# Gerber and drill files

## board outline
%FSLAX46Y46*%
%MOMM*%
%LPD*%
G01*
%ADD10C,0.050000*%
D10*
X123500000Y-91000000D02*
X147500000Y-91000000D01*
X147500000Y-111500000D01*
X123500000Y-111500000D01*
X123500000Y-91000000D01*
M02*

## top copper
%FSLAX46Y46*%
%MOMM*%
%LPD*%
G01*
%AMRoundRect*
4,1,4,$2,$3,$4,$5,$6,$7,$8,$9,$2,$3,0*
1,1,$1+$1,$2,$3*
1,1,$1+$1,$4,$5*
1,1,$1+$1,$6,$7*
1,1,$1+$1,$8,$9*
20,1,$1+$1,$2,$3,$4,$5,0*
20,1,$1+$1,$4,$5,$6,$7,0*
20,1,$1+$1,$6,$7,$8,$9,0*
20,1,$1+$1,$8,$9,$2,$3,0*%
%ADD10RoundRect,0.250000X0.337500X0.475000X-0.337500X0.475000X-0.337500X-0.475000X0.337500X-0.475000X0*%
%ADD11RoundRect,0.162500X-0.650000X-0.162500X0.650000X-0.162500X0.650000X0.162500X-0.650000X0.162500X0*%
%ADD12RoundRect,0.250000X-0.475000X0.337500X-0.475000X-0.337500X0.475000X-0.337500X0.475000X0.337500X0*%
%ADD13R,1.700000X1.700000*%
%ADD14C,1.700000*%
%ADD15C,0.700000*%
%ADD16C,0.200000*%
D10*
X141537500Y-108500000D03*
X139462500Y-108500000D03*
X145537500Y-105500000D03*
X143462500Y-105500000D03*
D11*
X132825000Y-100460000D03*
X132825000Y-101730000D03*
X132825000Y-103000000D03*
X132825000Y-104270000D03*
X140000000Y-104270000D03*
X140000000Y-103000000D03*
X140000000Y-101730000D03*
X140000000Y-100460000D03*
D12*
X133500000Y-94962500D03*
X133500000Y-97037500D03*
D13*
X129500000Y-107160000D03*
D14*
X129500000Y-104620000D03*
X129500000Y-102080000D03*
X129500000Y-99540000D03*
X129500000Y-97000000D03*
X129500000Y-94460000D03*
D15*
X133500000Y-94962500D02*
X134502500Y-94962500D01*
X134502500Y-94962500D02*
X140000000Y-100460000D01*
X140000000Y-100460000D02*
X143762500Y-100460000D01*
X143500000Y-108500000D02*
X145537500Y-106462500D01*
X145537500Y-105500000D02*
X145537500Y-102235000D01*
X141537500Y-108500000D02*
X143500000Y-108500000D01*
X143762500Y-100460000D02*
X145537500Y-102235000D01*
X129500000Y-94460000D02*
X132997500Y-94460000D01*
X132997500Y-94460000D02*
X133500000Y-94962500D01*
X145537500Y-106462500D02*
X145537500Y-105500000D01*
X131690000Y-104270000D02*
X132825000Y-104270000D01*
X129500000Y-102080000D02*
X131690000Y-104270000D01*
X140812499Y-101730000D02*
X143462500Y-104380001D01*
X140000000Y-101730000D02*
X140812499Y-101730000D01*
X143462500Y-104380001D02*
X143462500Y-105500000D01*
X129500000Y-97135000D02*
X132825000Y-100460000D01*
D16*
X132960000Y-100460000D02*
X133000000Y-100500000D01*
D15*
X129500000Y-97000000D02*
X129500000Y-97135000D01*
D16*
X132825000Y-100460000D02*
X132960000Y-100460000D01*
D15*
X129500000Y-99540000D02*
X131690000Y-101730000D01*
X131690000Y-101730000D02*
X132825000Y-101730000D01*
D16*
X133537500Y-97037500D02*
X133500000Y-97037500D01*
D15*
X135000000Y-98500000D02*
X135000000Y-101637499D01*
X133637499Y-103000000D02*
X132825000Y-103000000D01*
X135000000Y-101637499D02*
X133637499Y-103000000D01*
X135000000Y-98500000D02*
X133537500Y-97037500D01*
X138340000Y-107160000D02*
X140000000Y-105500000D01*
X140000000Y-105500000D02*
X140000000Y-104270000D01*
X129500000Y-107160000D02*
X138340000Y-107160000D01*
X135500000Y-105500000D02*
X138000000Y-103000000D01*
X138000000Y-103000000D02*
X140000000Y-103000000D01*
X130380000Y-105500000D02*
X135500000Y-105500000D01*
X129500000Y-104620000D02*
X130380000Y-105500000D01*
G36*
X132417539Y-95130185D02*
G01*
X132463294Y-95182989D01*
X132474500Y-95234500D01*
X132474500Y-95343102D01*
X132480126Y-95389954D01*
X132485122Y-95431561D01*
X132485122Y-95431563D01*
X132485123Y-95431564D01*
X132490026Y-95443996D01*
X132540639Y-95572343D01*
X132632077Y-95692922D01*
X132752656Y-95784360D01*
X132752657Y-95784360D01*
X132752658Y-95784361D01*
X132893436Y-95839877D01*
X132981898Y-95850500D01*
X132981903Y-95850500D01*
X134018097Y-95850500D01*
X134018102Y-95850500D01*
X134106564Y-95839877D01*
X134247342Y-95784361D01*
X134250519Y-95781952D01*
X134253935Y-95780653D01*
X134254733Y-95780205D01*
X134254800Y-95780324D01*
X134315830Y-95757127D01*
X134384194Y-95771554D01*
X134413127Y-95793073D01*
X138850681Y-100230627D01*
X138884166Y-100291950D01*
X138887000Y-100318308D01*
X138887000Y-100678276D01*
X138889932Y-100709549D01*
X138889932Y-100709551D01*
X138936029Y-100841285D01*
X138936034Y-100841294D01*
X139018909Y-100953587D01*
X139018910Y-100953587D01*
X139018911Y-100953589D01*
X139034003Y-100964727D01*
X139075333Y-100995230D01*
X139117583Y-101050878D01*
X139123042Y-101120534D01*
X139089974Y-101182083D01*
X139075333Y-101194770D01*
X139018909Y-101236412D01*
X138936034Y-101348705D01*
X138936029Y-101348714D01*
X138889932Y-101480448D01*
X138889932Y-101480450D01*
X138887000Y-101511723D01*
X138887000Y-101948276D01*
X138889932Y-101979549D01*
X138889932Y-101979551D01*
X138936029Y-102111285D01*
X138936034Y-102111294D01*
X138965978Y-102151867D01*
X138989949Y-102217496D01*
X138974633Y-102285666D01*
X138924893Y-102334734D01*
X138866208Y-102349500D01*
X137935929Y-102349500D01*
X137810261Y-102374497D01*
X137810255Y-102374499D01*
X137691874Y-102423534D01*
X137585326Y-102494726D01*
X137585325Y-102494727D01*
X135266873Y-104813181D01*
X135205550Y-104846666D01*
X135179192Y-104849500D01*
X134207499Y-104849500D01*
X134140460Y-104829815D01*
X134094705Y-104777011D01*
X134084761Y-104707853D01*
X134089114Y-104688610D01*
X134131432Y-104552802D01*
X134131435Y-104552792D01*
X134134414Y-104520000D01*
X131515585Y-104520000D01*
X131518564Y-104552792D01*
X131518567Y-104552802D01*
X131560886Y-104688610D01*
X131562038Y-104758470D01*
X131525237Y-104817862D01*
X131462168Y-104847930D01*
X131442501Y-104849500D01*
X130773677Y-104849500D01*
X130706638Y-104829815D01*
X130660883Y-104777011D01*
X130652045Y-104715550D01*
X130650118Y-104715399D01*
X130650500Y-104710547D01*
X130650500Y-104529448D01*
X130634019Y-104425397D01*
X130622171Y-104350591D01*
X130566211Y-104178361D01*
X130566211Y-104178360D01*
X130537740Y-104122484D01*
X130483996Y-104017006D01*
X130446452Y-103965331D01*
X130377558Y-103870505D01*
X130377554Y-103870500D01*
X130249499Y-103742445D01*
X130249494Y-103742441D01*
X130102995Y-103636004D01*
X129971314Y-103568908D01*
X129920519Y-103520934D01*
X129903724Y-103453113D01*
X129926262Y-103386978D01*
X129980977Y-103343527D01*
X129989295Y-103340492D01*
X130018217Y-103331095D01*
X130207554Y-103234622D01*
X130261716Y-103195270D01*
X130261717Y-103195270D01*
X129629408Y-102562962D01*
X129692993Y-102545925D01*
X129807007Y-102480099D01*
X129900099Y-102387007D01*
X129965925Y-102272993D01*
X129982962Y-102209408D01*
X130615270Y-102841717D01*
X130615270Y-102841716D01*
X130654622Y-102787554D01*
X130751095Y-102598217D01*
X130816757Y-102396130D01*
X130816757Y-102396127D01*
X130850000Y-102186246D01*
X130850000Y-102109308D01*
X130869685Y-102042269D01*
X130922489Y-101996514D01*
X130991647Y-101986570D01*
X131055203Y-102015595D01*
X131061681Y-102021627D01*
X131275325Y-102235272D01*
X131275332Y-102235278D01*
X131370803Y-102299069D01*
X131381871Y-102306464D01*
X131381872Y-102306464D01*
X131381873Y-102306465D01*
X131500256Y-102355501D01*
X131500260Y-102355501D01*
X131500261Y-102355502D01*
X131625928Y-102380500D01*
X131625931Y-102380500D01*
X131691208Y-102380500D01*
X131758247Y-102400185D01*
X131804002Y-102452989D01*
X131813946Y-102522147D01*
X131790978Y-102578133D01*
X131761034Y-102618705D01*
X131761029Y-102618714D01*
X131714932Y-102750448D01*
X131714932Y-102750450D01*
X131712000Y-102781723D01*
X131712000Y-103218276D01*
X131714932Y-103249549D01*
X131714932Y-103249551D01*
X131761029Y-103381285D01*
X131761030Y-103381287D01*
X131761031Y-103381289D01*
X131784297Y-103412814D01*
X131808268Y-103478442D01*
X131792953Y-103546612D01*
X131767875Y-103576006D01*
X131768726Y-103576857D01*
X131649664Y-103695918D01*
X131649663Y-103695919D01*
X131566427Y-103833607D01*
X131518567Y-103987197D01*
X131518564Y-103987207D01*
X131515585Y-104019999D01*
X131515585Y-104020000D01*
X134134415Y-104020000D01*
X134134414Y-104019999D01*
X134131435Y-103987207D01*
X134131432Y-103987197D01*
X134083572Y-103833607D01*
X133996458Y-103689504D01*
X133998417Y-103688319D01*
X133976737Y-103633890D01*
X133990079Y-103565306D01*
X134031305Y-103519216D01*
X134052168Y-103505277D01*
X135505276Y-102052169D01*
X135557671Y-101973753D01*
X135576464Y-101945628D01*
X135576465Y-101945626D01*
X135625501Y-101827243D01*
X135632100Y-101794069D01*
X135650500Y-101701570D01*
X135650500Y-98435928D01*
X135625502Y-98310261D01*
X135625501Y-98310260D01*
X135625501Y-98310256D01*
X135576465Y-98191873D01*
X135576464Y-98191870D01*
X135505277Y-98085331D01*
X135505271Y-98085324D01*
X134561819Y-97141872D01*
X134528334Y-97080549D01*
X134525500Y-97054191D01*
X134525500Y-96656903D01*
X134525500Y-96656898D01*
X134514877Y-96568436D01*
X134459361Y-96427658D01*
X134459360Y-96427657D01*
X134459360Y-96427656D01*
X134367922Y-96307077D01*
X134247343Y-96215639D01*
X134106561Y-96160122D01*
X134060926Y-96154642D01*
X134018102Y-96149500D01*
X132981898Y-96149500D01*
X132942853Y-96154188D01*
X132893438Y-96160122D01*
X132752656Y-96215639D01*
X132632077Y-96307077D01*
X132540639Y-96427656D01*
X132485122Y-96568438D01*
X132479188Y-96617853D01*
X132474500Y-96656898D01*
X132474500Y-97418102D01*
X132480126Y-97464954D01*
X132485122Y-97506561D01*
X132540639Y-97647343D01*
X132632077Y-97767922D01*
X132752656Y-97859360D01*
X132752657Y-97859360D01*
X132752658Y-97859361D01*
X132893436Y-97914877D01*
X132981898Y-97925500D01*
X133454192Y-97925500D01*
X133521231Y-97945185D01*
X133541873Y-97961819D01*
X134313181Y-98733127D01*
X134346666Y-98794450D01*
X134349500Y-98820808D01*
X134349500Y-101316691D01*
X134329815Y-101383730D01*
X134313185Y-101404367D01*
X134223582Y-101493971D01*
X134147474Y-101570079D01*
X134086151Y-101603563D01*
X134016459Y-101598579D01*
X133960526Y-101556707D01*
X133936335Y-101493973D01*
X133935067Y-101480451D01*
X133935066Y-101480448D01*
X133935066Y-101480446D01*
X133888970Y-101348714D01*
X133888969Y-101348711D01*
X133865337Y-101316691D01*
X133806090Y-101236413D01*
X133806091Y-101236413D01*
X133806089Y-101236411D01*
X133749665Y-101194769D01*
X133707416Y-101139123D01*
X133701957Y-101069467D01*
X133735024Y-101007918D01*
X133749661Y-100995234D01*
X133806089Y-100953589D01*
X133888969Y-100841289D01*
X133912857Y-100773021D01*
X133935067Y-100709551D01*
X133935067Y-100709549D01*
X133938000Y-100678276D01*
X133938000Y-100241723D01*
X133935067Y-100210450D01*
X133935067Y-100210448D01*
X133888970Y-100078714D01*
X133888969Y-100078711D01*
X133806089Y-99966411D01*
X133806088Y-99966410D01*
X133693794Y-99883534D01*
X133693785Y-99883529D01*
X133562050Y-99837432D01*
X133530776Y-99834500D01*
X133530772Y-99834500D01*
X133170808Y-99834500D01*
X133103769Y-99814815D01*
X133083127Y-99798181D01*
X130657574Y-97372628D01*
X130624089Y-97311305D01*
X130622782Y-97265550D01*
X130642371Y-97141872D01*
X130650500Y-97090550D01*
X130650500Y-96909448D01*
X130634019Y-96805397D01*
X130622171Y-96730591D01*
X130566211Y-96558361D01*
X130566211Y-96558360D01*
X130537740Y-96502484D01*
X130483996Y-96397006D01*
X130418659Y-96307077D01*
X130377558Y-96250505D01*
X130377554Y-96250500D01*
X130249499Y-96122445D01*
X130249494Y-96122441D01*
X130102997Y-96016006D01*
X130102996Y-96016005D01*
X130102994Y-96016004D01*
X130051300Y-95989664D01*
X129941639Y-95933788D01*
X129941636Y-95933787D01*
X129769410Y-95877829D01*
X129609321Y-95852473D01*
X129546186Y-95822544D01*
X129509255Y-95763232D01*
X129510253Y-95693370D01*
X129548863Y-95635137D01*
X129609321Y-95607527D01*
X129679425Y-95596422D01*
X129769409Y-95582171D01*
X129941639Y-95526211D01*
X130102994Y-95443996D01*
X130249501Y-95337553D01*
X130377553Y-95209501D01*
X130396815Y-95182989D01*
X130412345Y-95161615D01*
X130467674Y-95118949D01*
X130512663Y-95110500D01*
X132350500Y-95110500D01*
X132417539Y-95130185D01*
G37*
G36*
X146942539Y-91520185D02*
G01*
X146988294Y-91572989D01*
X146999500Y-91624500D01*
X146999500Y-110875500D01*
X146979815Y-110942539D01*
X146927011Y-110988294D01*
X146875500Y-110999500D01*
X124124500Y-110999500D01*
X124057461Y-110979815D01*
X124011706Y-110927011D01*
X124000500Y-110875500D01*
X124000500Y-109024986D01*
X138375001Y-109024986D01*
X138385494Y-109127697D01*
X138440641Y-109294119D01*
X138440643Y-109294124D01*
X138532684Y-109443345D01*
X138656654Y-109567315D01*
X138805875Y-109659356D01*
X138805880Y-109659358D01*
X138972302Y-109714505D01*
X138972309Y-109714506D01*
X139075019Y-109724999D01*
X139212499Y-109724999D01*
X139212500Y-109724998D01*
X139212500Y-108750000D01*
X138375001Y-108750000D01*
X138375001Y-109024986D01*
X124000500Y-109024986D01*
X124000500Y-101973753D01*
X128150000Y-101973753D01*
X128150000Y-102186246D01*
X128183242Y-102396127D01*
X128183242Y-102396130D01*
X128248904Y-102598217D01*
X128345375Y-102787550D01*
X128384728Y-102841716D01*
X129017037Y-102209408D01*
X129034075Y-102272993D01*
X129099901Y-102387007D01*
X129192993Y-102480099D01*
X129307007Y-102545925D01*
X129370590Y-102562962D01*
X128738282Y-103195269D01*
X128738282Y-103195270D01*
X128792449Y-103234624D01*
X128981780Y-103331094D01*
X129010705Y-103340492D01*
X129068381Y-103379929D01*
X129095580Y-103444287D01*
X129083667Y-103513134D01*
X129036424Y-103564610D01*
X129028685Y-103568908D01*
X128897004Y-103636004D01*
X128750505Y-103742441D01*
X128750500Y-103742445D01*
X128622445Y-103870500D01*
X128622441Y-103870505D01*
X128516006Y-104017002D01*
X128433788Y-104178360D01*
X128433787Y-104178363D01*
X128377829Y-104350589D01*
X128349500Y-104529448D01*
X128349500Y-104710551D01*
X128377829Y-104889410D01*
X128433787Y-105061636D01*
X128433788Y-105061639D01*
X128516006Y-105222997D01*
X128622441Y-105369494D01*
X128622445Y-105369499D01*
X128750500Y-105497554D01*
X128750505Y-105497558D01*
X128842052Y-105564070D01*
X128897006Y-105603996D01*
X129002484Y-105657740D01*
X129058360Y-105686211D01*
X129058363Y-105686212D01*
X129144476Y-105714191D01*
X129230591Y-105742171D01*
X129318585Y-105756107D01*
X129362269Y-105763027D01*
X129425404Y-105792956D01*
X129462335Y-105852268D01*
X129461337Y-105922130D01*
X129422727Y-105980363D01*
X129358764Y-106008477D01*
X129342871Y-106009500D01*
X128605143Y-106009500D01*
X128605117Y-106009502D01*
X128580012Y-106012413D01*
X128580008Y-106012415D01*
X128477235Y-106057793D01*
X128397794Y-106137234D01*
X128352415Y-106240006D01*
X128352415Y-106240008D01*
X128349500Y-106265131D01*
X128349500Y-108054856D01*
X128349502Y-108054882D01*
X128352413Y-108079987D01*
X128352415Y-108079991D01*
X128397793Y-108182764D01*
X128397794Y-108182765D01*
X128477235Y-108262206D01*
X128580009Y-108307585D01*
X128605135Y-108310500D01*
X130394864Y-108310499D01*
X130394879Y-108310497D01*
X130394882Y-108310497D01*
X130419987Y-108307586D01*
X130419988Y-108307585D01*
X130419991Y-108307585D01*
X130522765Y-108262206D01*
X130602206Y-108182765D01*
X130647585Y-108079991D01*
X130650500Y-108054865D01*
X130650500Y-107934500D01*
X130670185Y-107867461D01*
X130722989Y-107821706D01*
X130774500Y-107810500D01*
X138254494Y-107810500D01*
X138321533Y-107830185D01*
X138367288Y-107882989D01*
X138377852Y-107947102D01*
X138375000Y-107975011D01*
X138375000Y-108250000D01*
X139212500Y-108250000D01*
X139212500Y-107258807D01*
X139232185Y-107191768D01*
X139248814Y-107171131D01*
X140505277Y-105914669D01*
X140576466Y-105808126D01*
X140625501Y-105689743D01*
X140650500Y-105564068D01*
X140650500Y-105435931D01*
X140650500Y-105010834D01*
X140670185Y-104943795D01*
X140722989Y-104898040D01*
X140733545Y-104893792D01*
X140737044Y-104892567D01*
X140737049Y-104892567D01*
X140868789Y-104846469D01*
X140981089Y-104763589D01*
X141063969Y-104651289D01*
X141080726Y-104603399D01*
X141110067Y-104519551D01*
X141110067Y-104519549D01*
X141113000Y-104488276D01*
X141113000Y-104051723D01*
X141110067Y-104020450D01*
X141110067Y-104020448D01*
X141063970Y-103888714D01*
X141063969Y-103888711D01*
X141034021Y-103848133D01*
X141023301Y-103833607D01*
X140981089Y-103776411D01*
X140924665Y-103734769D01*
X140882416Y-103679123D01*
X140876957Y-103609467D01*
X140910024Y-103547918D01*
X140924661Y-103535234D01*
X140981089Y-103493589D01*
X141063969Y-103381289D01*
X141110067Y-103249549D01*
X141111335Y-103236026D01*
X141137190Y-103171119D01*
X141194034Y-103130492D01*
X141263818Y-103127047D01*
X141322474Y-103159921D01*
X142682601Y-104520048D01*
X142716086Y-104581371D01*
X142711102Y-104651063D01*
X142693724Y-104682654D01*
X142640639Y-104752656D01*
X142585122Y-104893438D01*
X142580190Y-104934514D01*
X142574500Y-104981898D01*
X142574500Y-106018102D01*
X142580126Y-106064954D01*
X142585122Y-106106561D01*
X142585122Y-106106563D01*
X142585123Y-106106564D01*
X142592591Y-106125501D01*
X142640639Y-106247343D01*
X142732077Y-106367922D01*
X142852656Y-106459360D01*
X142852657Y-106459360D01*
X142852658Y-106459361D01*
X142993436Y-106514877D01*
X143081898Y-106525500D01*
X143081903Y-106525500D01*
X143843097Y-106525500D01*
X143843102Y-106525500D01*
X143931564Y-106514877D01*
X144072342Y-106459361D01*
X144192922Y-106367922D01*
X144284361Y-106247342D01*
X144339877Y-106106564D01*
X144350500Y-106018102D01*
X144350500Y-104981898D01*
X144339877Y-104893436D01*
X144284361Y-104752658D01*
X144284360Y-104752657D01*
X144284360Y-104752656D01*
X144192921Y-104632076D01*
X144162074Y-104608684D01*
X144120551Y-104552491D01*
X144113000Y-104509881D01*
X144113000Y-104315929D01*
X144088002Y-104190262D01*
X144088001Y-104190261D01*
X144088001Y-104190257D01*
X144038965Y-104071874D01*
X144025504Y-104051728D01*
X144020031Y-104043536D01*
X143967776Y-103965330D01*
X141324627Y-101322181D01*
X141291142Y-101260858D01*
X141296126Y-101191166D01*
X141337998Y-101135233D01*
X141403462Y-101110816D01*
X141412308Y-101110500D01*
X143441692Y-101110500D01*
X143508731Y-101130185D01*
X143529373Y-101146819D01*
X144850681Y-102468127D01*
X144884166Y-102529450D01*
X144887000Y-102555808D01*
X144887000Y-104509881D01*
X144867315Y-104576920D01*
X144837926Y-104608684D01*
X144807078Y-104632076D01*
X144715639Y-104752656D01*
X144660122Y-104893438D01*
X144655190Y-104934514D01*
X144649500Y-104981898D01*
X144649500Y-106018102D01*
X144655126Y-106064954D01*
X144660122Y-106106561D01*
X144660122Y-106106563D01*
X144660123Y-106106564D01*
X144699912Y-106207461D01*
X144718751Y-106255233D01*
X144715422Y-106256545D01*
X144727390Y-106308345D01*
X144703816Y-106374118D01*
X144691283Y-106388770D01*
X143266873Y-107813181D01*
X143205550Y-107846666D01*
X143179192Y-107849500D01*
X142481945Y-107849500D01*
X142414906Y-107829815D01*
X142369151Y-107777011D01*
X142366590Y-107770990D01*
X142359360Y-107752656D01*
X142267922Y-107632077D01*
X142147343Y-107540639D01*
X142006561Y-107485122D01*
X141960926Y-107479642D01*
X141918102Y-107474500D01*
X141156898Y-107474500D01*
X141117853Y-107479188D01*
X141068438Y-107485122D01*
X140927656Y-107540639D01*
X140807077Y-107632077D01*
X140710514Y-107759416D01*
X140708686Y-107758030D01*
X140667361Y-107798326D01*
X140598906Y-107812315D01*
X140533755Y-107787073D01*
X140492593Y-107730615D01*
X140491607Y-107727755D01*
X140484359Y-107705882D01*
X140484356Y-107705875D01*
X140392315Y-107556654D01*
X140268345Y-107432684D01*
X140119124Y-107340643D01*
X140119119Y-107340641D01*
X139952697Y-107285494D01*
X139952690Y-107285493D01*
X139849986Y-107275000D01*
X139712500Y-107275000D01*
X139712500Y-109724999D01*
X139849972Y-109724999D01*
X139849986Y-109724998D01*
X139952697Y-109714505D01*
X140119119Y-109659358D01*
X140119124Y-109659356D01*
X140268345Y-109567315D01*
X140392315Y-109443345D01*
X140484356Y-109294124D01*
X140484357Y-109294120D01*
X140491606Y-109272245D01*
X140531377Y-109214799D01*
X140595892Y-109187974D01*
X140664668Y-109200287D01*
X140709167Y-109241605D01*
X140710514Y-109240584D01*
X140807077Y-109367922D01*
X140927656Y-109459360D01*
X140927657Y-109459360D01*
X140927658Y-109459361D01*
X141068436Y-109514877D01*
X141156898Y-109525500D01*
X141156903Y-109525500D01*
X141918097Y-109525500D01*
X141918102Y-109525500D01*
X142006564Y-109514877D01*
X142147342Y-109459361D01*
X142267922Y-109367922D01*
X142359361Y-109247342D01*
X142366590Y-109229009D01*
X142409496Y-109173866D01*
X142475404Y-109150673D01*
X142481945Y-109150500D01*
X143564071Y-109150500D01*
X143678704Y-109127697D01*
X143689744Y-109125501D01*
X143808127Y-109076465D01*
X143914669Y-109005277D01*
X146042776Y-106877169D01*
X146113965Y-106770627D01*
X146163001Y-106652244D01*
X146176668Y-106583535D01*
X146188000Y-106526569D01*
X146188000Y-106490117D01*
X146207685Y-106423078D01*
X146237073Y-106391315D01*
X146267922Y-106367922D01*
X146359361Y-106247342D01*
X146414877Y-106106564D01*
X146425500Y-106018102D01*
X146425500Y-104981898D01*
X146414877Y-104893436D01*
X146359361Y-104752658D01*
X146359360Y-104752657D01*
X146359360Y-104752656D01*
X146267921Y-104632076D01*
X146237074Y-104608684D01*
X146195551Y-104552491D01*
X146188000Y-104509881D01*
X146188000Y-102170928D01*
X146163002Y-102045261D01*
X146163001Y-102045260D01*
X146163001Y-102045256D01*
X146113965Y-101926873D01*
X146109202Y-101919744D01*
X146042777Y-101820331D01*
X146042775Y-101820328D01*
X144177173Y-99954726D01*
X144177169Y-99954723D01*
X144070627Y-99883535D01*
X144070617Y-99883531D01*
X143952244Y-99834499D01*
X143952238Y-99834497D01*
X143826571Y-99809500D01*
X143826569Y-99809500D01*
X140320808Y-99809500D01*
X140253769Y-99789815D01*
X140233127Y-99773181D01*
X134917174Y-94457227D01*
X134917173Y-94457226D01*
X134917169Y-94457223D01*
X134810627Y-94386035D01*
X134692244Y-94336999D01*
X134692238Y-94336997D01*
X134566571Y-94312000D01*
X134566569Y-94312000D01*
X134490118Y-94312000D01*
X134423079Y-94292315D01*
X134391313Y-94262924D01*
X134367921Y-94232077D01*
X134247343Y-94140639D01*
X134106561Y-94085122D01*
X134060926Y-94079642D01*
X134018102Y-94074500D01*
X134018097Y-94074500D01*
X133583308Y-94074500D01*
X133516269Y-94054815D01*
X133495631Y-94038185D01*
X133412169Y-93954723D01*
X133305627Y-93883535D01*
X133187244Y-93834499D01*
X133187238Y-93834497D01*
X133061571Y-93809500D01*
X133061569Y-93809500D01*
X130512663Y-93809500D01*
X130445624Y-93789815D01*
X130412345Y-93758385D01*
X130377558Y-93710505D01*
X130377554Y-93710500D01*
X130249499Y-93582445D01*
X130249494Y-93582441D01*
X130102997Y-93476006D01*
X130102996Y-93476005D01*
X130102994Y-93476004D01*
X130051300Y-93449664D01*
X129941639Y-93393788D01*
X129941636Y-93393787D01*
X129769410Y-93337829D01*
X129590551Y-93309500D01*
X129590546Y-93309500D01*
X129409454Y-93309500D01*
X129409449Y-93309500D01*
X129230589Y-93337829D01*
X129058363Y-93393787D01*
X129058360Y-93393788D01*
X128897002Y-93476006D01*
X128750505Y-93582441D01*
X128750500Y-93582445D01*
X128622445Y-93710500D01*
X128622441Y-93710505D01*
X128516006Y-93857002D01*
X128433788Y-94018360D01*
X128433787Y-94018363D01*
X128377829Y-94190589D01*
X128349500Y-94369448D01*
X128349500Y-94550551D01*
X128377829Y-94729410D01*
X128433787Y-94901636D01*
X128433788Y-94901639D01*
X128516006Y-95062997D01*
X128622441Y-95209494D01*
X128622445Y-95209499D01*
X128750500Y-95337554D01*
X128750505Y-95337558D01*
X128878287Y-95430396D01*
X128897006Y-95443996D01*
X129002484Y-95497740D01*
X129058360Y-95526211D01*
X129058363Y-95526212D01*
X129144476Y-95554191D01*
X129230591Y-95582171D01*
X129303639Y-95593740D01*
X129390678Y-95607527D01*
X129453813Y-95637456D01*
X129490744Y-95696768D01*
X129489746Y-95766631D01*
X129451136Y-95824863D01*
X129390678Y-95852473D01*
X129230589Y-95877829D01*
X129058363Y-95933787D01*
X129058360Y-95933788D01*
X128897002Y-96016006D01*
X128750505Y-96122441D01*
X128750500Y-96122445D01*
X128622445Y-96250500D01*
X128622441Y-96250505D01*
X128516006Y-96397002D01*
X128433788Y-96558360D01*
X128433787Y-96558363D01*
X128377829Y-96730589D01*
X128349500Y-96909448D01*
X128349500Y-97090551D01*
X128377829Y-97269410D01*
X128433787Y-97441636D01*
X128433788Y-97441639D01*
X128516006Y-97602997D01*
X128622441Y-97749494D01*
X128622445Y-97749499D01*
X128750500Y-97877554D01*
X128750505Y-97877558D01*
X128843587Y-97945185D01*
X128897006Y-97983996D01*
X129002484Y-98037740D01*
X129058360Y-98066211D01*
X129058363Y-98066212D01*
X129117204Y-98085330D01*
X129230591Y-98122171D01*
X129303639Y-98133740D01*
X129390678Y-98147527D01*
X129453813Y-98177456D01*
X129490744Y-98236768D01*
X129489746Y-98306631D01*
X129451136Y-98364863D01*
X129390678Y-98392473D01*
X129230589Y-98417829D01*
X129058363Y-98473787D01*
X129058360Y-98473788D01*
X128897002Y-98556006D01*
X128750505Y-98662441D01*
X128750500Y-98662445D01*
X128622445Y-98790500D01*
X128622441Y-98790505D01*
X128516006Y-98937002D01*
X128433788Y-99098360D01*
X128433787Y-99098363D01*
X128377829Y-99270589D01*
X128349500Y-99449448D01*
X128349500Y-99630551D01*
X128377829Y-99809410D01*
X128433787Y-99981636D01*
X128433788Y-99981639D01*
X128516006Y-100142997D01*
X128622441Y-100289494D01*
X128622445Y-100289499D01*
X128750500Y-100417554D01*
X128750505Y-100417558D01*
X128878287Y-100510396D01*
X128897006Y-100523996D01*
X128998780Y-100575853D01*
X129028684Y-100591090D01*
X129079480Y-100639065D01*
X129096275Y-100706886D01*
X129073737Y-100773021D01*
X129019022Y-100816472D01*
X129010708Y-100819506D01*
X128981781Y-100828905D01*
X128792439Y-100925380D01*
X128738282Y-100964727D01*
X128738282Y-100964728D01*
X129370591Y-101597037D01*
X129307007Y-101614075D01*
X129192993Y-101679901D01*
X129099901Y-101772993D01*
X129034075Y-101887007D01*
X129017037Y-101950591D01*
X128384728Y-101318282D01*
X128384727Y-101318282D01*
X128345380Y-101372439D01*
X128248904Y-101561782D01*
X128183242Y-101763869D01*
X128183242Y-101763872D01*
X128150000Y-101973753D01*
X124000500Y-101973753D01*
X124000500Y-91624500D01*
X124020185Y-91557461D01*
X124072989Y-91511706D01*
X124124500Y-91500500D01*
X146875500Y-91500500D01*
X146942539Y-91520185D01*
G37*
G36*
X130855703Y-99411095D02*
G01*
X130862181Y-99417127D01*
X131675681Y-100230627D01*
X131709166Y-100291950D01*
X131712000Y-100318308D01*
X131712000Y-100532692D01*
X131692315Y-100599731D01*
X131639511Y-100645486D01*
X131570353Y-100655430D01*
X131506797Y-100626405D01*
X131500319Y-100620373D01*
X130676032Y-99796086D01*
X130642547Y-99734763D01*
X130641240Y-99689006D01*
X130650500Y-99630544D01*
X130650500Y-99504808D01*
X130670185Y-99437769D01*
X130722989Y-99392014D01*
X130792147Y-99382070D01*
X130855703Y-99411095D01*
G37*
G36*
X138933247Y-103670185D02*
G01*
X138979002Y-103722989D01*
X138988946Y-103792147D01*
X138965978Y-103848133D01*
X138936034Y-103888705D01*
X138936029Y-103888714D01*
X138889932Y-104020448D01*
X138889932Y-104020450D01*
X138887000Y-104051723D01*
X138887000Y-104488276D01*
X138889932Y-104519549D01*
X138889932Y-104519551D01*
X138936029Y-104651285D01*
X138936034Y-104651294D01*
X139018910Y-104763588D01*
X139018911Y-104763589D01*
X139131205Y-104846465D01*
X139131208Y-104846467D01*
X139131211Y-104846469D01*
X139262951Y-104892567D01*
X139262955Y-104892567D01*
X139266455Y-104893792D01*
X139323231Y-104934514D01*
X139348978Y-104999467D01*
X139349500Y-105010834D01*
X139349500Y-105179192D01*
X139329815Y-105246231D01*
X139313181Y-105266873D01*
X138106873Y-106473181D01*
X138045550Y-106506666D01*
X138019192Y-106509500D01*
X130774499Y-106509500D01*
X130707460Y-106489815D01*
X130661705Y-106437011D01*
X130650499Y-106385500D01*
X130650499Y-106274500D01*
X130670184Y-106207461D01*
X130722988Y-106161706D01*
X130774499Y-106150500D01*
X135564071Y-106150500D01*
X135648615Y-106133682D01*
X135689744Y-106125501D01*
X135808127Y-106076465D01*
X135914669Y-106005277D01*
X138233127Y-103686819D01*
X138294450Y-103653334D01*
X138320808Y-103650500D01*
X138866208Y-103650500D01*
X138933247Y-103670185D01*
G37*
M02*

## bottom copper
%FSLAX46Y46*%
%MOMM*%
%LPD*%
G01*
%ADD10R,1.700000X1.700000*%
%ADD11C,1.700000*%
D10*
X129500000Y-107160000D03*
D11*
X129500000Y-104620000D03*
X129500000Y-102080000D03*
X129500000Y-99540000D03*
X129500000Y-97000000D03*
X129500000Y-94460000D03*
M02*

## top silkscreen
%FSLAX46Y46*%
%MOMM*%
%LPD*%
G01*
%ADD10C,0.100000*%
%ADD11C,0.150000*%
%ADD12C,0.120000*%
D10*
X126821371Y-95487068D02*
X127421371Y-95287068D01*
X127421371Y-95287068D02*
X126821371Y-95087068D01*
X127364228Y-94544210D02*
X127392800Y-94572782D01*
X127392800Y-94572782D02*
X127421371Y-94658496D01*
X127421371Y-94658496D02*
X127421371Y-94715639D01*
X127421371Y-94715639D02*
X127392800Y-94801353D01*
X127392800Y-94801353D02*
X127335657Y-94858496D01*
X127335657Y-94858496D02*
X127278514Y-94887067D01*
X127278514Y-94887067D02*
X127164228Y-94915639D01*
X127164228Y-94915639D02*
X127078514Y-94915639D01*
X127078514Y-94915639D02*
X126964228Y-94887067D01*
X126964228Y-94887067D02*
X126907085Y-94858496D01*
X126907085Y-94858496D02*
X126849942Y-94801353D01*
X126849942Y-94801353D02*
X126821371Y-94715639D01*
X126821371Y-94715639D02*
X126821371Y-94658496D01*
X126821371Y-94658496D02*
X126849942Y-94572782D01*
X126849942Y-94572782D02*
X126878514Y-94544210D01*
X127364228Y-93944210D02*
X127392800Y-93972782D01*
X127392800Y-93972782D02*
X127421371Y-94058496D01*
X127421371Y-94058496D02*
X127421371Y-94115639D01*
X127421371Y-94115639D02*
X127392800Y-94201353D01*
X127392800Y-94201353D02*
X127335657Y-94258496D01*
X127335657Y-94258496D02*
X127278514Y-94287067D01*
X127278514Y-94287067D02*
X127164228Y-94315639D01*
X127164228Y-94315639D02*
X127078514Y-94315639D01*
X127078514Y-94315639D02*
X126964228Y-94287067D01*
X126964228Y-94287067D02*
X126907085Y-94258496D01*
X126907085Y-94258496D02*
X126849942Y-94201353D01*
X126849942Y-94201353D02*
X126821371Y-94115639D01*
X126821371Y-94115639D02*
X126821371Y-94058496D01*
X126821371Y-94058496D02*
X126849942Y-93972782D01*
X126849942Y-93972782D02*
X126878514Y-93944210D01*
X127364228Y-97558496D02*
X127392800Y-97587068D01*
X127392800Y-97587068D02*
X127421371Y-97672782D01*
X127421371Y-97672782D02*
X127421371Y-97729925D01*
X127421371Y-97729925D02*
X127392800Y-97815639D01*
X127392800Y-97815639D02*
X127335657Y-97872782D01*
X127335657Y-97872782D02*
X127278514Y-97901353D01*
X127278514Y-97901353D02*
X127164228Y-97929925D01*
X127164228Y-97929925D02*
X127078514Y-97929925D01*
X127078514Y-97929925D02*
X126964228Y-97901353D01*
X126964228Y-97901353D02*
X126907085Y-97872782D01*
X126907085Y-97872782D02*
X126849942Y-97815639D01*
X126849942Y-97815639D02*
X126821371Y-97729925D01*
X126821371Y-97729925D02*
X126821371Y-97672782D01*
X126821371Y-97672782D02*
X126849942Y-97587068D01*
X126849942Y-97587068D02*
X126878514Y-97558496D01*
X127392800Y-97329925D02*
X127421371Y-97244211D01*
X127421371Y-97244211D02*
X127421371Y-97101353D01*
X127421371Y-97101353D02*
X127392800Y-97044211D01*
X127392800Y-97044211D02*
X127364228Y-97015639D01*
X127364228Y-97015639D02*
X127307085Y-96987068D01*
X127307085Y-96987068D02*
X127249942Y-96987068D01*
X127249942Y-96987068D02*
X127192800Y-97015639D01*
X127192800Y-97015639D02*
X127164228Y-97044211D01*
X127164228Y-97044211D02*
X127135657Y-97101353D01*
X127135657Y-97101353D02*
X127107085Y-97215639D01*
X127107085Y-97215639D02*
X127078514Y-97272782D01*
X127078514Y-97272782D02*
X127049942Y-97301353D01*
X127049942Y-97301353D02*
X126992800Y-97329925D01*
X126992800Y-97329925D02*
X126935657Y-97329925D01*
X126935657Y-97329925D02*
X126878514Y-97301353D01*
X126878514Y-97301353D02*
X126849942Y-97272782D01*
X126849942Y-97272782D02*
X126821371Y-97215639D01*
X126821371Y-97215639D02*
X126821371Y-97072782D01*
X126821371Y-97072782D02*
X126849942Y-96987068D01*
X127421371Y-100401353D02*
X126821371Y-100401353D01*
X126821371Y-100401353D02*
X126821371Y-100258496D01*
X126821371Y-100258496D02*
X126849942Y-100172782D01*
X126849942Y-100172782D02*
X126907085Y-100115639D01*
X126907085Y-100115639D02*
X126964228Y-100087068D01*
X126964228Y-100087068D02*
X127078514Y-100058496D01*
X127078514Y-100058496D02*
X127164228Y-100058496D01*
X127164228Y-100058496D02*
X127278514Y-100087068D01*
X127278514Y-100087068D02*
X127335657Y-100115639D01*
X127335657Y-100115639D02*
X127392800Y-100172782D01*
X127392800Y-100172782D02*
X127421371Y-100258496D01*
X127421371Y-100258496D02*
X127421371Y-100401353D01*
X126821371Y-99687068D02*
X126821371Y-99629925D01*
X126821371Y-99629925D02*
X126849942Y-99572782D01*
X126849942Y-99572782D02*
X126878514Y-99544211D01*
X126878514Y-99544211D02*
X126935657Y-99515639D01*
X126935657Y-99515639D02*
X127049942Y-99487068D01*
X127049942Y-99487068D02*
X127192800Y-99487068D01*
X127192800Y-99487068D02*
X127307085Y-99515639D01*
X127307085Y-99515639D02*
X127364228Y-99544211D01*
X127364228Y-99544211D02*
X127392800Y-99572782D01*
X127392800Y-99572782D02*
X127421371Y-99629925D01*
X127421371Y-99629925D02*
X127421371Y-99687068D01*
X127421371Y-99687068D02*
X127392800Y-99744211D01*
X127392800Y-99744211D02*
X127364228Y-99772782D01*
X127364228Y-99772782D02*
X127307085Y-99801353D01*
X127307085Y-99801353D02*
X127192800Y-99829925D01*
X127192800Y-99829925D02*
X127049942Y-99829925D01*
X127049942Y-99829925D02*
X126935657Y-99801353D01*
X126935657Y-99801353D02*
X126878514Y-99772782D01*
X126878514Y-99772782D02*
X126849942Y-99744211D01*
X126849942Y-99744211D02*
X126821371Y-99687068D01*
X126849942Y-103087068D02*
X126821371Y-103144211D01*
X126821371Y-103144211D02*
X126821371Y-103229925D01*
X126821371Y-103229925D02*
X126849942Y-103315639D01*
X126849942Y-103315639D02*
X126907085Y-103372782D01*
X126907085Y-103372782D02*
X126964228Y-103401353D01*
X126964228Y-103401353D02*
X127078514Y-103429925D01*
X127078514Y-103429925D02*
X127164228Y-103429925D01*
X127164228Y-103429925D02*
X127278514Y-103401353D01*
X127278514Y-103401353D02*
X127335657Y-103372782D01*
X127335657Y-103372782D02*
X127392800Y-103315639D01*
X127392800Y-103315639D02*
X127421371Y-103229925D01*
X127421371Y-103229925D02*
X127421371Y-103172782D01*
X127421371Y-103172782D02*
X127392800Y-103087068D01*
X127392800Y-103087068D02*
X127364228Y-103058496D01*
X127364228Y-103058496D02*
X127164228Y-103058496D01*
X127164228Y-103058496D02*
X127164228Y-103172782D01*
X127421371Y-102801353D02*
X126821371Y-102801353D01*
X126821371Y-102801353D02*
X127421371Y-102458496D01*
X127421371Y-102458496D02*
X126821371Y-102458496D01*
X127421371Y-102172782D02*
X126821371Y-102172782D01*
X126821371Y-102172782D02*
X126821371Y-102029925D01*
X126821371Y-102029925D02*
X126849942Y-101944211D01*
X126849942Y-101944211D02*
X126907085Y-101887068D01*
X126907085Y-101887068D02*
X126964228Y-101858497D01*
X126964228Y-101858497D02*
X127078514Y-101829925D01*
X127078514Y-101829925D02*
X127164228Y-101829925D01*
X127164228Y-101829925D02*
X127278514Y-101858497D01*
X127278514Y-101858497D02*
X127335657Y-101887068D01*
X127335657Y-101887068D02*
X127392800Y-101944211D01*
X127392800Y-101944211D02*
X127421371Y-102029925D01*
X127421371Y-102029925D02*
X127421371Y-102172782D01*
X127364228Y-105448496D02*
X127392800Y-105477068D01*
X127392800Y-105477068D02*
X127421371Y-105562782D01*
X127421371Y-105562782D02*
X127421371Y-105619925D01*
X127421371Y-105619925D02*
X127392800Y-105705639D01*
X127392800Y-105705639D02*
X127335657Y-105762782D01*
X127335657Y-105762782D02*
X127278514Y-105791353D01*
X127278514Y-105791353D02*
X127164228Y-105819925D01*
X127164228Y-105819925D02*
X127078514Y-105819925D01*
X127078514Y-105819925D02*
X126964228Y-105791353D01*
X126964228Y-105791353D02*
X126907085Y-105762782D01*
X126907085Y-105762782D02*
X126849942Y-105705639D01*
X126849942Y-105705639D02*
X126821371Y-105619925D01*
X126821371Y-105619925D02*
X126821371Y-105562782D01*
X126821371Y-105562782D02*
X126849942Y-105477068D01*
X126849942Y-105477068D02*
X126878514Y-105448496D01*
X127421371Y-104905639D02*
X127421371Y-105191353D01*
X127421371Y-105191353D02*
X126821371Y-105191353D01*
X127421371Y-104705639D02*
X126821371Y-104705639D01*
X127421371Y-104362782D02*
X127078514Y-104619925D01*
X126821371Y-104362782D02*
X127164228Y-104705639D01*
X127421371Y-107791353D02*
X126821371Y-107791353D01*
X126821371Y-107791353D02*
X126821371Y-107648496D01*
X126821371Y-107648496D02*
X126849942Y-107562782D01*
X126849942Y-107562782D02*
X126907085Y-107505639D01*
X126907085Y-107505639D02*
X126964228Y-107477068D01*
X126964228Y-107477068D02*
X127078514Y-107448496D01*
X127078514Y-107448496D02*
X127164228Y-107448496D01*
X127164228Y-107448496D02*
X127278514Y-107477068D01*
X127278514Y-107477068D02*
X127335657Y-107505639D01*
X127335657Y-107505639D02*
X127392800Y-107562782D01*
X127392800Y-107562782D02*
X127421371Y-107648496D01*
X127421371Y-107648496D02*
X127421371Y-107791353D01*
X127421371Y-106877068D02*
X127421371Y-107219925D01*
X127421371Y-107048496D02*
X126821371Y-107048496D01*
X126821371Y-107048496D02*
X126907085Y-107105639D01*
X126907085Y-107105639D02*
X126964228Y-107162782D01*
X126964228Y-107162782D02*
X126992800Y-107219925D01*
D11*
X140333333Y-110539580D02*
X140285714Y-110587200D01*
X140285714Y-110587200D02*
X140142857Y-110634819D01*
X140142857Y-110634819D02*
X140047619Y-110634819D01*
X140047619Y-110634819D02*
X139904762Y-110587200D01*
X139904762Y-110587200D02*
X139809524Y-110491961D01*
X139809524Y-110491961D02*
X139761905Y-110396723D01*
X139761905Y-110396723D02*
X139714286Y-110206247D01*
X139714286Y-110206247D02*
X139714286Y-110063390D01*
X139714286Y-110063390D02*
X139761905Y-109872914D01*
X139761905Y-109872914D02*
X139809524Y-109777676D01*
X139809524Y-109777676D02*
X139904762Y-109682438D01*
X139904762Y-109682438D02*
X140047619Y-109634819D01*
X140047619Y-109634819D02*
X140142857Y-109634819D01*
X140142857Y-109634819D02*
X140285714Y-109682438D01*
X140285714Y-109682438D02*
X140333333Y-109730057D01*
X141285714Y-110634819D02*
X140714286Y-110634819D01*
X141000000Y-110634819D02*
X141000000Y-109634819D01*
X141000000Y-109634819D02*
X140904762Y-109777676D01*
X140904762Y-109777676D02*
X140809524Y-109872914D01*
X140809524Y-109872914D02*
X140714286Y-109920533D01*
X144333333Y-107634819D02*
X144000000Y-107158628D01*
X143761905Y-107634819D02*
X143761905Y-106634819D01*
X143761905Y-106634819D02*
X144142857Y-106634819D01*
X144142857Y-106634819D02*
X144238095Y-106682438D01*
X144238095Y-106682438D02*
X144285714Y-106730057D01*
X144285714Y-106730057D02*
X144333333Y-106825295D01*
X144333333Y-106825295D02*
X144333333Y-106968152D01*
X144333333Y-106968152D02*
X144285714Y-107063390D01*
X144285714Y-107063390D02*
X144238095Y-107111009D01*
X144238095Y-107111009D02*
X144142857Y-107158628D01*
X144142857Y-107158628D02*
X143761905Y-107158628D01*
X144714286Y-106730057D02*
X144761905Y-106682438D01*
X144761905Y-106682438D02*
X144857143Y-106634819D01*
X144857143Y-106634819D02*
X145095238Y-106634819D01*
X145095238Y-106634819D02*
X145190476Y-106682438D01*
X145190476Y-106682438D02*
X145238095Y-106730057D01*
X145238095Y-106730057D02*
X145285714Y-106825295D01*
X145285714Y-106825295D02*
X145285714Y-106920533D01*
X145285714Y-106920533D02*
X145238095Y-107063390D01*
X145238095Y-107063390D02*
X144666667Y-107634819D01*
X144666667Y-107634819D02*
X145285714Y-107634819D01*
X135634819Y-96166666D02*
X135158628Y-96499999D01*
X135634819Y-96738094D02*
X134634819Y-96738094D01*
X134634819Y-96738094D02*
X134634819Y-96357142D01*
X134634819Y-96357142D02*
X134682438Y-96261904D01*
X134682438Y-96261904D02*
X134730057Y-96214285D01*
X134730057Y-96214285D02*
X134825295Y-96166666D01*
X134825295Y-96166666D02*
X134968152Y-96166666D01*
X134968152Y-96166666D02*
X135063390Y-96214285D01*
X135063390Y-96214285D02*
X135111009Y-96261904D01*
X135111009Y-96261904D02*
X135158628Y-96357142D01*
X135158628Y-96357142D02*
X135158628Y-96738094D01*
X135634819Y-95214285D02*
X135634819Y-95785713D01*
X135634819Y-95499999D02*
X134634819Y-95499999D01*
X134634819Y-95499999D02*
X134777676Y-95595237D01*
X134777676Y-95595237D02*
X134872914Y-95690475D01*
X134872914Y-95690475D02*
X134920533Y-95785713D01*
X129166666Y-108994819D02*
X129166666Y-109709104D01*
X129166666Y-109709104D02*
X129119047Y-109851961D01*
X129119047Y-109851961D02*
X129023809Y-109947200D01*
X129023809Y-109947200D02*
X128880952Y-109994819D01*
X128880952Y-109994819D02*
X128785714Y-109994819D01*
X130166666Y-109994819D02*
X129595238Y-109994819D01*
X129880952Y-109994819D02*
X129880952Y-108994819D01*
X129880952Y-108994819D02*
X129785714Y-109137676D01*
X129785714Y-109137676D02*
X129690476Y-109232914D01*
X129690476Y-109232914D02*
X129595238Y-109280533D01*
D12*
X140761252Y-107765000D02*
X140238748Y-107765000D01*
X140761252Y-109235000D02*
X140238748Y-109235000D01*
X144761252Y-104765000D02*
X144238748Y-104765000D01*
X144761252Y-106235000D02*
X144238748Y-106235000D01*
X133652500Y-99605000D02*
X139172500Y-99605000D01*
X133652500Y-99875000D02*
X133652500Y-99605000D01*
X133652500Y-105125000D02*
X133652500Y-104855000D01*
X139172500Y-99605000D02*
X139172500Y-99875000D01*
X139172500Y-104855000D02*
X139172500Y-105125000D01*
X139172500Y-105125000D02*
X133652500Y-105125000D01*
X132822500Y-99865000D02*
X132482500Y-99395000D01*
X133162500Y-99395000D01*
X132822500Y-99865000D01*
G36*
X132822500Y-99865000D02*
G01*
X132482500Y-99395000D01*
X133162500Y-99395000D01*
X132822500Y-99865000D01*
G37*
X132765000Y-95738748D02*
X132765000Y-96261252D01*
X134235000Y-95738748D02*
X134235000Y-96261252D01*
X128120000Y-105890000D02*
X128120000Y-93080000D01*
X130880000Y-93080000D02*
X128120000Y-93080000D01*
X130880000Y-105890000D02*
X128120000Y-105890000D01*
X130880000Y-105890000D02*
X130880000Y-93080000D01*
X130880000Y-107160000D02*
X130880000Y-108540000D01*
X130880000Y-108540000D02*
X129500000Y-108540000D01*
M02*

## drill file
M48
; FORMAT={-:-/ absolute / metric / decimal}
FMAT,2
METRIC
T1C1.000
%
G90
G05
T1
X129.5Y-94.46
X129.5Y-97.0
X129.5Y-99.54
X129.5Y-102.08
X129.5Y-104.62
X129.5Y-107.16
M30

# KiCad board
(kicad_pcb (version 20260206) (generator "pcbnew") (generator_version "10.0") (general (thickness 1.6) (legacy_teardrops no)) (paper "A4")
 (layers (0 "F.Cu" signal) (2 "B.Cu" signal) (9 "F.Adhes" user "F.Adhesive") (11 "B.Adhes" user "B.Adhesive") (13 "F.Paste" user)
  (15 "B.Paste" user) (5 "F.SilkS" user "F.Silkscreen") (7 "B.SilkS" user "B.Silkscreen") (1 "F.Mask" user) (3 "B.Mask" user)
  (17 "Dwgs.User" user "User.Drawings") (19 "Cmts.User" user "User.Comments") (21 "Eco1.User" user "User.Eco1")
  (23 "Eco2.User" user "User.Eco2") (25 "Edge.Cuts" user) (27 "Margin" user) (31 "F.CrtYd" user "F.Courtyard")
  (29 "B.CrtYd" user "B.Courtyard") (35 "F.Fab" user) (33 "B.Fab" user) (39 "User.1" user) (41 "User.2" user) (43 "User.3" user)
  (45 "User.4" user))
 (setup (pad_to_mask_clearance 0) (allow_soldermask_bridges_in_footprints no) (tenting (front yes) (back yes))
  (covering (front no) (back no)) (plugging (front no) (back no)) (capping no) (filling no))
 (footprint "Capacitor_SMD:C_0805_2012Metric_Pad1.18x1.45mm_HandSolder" (layer "F.Cu") (at 140.5 108.5 180)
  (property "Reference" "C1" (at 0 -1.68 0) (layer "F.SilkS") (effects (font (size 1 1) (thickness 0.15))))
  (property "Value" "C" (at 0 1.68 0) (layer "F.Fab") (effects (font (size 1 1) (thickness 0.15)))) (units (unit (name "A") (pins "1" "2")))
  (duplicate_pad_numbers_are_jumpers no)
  (fp_line (start -0.261252 0.735) (end 0.261252 0.735) (stroke (width 0.12) (type solid)) (layer "F.SilkS"))
  (fp_line (start -0.261252 -0.735) (end 0.261252 -0.735) (stroke (width 0.12) (type solid)) (layer "F.SilkS"))
  (pad "1" smd roundrect (at -1.0375 0 180) (size 1.175 1.45) (layers "F.Cu" "F.Mask" "F.Paste") (roundrect_rratio 0.212766) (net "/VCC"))
  (pad "2" smd roundrect (at 1.0375 0 180) (size 1.175 1.45) (layers "F.Cu" "F.Mask" "F.Paste") (roundrect_rratio 0.212766) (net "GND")))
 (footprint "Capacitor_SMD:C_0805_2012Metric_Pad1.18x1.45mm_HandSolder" (layer "F.Cu") (at 144.5 105.5 180)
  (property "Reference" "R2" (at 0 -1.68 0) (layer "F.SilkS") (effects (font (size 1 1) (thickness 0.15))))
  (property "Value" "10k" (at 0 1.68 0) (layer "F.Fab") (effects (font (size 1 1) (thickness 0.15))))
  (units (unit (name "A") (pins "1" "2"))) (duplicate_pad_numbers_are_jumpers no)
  (fp_line (start -0.261252 0.735) (end 0.261252 0.735) (stroke (width 0.12) (type solid)) (layer "F.SilkS"))
  (fp_line (start -0.261252 -0.735) (end 0.261252 -0.735) (stroke (width 0.12) (type solid)) (layer "F.SilkS"))
  (pad "1" smd roundrect (at -1.0375 0 180) (size 1.175 1.45) (layers "F.Cu" "F.Mask" "F.Paste") (roundrect_rratio 0.212766) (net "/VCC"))
  (pad "2" smd roundrect (at 1.0375 0 180) (size 1.175 1.45) (layers "F.Cu" "F.Mask" "F.Paste") (roundrect_rratio 0.212766) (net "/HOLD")))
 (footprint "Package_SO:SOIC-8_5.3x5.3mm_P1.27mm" (layer "F.Cu") (at 136.4125 102.365)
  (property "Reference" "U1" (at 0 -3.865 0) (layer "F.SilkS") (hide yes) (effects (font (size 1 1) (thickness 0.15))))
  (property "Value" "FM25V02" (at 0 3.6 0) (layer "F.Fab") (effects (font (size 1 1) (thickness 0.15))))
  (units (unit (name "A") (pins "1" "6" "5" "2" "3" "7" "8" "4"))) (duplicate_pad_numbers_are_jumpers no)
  (fp_line (start -2.76 -2.76) (end 2.76 -2.76) (stroke (width 0.12) (type solid)) (layer "F.SilkS"))
  (fp_line (start -2.76 -2.49) (end -2.76 -2.76) (stroke (width 0.12) (type solid)) (layer "F.SilkS"))
  (fp_line (start -2.76 2.76) (end -2.76 2.49) (stroke (width 0.12) (type solid)) (layer "F.SilkS"))
  (fp_line (start 2.76 -2.76) (end 2.76 -2.49) (stroke (width 0.12) (type solid)) (layer "F.SilkS"))
  (fp_line (start 2.76 2.49) (end 2.76 2.76) (stroke (width 0.12) (type solid)) (layer "F.SilkS"))
  (fp_line (start 2.76 2.76) (end -2.76 2.76) (stroke (width 0.12) (type solid)) (layer "F.SilkS"))
  (fp_poly (pts (xy -3.59 -2.5) (xy -3.93 -2.97) (xy -3.25 -2.97)) (stroke (width 0.12) (type solid)) (fill yes) (layer "F.SilkS"))
  (pad "1" smd roundrect (at -3.5875 -1.905) (size 1.625 0.65) (layers "F.Cu" "F.Mask" "F.Paste") (roundrect_rratio 0.25) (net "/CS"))
  (pad "2" smd roundrect (at -3.5875 -0.635) (size 1.625 0.65) (layers "F.Cu" "F.Mask" "F.Paste") (roundrect_rratio 0.25) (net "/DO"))
  (pad "3" smd roundrect (at -3.5875 0.635) (size 1.625 0.65) (layers "F.Cu" "F.Mask" "F.Paste") (roundrect_rratio 0.25) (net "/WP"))
  (pad "4" smd roundrect (at -3.5875 1.905) (size 1.625 0.65) (layers "F.Cu" "F.Mask" "F.Paste") (roundrect_rratio 0.25) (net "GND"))
  (pad "5" smd roundrect (at 3.5875 1.905) (size 1.625 0.65) (layers "F.Cu" "F.Mask" "F.Paste") (roundrect_rratio 0.25) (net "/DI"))
  (pad "6" smd roundrect (at 3.5875 0.635) (size 1.625 0.65) (layers "F.Cu" "F.Mask" "F.Paste") (roundrect_rratio 0.25) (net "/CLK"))
  (pad "7" smd roundrect (at 3.5875 -0.635) (size 1.625 0.65) (layers "F.Cu" "F.Mask" "F.Paste") (roundrect_rratio 0.25) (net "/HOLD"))
  (pad "8" smd roundrect (at 3.5875 -1.905) (size 1.625 0.65) (layers "F.Cu" "F.Mask" "F.Paste") (roundrect_rratio 0.25) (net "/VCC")))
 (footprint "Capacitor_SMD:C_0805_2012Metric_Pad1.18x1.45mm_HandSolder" (layer "F.Cu") (at 133.5 96 -90)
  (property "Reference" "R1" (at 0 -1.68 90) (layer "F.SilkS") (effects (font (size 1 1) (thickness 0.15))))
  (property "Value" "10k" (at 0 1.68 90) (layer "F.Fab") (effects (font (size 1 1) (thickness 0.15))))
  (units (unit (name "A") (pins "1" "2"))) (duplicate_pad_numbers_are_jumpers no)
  (fp_line (start -0.261252 0.735) (end 0.261252 0.735) (stroke (width 0.12) (type solid)) (layer "F.SilkS"))
  (fp_line (start -0.261252 -0.735) (end 0.261252 -0.735) (stroke (width 0.12) (type solid)) (layer "F.SilkS"))
  (pad "1" smd roundrect (at -1.0375 0 270) (size 1.175 1.45) (layers "F.Cu" "F.Mask" "F.Paste") (roundrect_rratio 0.212766) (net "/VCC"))
  (pad "2" smd roundrect (at 1.0375 0 270) (size 1.175 1.45) (layers "F.Cu" "F.Mask" "F.Paste") (roundrect_rratio 0.212766) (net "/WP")))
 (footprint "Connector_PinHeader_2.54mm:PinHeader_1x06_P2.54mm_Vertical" (layer "F.Cu") (at 129.5 107.16 180)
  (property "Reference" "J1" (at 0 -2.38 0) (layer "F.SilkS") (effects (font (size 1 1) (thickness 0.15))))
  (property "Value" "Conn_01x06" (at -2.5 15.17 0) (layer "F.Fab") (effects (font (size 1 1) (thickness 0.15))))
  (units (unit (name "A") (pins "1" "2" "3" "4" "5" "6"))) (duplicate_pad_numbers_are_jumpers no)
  (fp_line (start 1.38 1.27) (end 1.38 14.08) (stroke (width 0.12) (type solid)) (layer "F.SilkS"))
  (fp_line (start -1.38 14.08) (end 1.38 14.08) (stroke (width 0.12) (type solid)) (layer "F.SilkS"))
  (fp_line (start -1.38 1.27) (end 1.38 1.27) (stroke (width 0.12) (type solid)) (layer "F.SilkS"))
  (fp_line (start -1.38 1.27) (end -1.38 14.08) (stroke (width 0.12) (type solid)) (layer "F.SilkS"))
  (fp_line (start -1.38 0) (end -1.38 -1.38) (stroke (width 0.12) (type solid)) (layer "F.SilkS"))
  (fp_line (start -1.38 -1.38) (end 0 -1.38) (stroke (width 0.12) (type solid)) (layer "F.SilkS"))
  (pad "1" thru_hole rect (at 0 0 180) (size 1.7 1.7) (drill 1) (layers "*.Cu" "*.Mask") (remove_unused_layers no) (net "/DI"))
  (pad "2" thru_hole circle (at 0 2.54 180) (size 1.7 1.7) (drill 1) (layers "*.Cu" "*.Mask") (remove_unused_layers no) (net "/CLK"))
  (pad "3" thru_hole circle (at 0 5.08 180) (size 1.7 1.7) (drill 1) (layers "*.Cu" "*.Mask") (remove_unused_layers no) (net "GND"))
  (pad "4" thru_hole circle (at 0 7.62 180) (size 1.7 1.7) (drill 1) (layers "*.Cu" "*.Mask") (remove_unused_layers no) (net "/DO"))
  (pad "5" thru_hole circle (at 0 10.16 180) (size 1.7 1.7) (drill 1) (layers "*.Cu" "*.Mask") (remove_unused_layers no) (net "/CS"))
  (pad "6" thru_hole circle (at 0 12.7 180) (size 1.7 1.7) (drill 1) (layers "*.Cu" "*.Mask") (remove_unused_layers no) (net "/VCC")))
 (gr_rect (start 123.5 91) (end 147.5 111.5) (stroke (width 0.05) (type default)) (fill no) (layer "Edge.Cuts"))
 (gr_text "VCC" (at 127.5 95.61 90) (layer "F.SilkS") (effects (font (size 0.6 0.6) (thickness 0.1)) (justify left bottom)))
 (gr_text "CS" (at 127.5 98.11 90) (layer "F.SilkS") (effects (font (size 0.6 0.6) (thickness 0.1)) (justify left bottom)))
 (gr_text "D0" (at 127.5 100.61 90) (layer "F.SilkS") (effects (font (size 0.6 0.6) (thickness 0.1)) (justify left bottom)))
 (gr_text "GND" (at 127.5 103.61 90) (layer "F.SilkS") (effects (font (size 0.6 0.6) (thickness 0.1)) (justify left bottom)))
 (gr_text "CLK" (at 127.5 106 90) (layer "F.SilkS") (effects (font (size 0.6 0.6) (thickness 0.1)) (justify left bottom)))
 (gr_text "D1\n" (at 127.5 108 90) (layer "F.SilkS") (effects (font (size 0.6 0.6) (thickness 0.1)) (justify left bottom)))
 (segment (start 133.5 94.9625) (end 134.5025 94.9625) (width 0.7) (layer "F.Cu") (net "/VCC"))
 (segment (start 134.5025 94.9625) (end 140 100.46) (width 0.7) (layer "F.Cu") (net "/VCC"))
 (segment (start 140 100.46) (end 143.7625 100.46) (width 0.7) (layer "F.Cu") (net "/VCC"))
 (segment (start 143.5 108.5) (end 145.5375 106.4625) (width 0.7) (layer "F.Cu") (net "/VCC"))
 (segment (start 145.5375 105.5) (end 145.5375 102.235) (width 0.7) (layer "F.Cu") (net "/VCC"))
 (segment (start 141.5375 108.5) (end 143.5 108.5) (width 0.7) (layer "F.Cu") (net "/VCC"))
 (segment (start 143.7625 100.46) (end 145.5375 102.235) (width 0.7) (layer "F.Cu") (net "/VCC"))
 (segment (start 129.5 94.46) (end 132.9975 94.46) (width 0.7) (layer "F.Cu") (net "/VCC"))
 (segment (start 132.9975 94.46) (end 133.5 94.9625) (width 0.7) (layer "F.Cu") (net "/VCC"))
 (segment (start 145.5375 106.4625) (end 145.5375 105.5) (width 0.7) (layer "F.Cu") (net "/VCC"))
 (segment (start 131.69 104.27) (end 132.825 104.27) (width 0.7) (layer "F.Cu") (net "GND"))
 (segment (start 129.5 102.08) (end 131.69 104.27) (width 0.7) (layer "F.Cu") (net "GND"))
 (segment (start 140.812499 101.73) (end 143.4625 104.380001) (width 0.7) (layer "F.Cu") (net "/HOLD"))
 (segment (start 140 101.73) (end 140.812499 101.73) (width 0.7) (layer "F.Cu") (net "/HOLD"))
 (segment (start 143.4625 104.380001) (end 143.4625 105.5) (width 0.7) (layer "F.Cu") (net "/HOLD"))
 (segment (start 129.5 97.135) (end 132.825 100.46) (width 0.7) (layer "F.Cu") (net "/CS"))
 (segment (start 132.96 100.46) (end 133 100.5) (width 0.2) (layer "F.Cu") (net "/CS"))
 (segment (start 129.5 97) (end 129.5 97.135) (width 0.7) (layer "F.Cu") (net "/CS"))
 (segment (start 132.825 100.46) (end 132.96 100.46) (width 0.2) (layer "F.Cu") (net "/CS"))
 (segment (start 129.5 99.54) (end 131.69 101.73) (width 0.7) (layer "F.Cu") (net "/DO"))
 (segment (start 131.69 101.73) (end 132.825 101.73) (width 0.7) (layer "F.Cu") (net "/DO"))
 (segment (start 133.5375 97.0375) (end 133.5 97.0375) (width 0.2) (layer "F.Cu") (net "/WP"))
 (segment (start 135 98.5) (end 135 101.637499) (width 0.7) (layer "F.Cu") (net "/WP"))
 (segment (start 133.637499 103) (end 132.825 103) (width 0.7) (layer "F.Cu") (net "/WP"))
 (segment (start 135 101.637499) (end 133.637499 103) (width 0.7) (layer "F.Cu") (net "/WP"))
 (segment (start 135 98.5) (end 133.5375 97.0375) (width 0.7) (layer "F.Cu") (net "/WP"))
 (segment (start 138.34 107.16) (end 140 105.5) (width 0.7) (layer "F.Cu") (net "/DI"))
 (segment (start 140 105.5) (end 140 104.27) (width 0.7) (layer "F.Cu") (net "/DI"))
 (segment (start 129.5 107.16) (end 138.34 107.16) (width 0.7) (layer "F.Cu") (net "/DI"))
 (segment (start 135.5 105.5) (end 138 103) (width 0.7) (layer "F.Cu") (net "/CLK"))
 (segment (start 138 103) (end 140 103) (width 0.7) (layer "F.Cu") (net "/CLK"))
 (segment (start 130.38 105.5) (end 135.5 105.5) (width 0.7) (layer "F.Cu") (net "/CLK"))
 (segment (start 129.5 104.62) (end 130.38 105.5) (width 0.7) (layer "F.Cu") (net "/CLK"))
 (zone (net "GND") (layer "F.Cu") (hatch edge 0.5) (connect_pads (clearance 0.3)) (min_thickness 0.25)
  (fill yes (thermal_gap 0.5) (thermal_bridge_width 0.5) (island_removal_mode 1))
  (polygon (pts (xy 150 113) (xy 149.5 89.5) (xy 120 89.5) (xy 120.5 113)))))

